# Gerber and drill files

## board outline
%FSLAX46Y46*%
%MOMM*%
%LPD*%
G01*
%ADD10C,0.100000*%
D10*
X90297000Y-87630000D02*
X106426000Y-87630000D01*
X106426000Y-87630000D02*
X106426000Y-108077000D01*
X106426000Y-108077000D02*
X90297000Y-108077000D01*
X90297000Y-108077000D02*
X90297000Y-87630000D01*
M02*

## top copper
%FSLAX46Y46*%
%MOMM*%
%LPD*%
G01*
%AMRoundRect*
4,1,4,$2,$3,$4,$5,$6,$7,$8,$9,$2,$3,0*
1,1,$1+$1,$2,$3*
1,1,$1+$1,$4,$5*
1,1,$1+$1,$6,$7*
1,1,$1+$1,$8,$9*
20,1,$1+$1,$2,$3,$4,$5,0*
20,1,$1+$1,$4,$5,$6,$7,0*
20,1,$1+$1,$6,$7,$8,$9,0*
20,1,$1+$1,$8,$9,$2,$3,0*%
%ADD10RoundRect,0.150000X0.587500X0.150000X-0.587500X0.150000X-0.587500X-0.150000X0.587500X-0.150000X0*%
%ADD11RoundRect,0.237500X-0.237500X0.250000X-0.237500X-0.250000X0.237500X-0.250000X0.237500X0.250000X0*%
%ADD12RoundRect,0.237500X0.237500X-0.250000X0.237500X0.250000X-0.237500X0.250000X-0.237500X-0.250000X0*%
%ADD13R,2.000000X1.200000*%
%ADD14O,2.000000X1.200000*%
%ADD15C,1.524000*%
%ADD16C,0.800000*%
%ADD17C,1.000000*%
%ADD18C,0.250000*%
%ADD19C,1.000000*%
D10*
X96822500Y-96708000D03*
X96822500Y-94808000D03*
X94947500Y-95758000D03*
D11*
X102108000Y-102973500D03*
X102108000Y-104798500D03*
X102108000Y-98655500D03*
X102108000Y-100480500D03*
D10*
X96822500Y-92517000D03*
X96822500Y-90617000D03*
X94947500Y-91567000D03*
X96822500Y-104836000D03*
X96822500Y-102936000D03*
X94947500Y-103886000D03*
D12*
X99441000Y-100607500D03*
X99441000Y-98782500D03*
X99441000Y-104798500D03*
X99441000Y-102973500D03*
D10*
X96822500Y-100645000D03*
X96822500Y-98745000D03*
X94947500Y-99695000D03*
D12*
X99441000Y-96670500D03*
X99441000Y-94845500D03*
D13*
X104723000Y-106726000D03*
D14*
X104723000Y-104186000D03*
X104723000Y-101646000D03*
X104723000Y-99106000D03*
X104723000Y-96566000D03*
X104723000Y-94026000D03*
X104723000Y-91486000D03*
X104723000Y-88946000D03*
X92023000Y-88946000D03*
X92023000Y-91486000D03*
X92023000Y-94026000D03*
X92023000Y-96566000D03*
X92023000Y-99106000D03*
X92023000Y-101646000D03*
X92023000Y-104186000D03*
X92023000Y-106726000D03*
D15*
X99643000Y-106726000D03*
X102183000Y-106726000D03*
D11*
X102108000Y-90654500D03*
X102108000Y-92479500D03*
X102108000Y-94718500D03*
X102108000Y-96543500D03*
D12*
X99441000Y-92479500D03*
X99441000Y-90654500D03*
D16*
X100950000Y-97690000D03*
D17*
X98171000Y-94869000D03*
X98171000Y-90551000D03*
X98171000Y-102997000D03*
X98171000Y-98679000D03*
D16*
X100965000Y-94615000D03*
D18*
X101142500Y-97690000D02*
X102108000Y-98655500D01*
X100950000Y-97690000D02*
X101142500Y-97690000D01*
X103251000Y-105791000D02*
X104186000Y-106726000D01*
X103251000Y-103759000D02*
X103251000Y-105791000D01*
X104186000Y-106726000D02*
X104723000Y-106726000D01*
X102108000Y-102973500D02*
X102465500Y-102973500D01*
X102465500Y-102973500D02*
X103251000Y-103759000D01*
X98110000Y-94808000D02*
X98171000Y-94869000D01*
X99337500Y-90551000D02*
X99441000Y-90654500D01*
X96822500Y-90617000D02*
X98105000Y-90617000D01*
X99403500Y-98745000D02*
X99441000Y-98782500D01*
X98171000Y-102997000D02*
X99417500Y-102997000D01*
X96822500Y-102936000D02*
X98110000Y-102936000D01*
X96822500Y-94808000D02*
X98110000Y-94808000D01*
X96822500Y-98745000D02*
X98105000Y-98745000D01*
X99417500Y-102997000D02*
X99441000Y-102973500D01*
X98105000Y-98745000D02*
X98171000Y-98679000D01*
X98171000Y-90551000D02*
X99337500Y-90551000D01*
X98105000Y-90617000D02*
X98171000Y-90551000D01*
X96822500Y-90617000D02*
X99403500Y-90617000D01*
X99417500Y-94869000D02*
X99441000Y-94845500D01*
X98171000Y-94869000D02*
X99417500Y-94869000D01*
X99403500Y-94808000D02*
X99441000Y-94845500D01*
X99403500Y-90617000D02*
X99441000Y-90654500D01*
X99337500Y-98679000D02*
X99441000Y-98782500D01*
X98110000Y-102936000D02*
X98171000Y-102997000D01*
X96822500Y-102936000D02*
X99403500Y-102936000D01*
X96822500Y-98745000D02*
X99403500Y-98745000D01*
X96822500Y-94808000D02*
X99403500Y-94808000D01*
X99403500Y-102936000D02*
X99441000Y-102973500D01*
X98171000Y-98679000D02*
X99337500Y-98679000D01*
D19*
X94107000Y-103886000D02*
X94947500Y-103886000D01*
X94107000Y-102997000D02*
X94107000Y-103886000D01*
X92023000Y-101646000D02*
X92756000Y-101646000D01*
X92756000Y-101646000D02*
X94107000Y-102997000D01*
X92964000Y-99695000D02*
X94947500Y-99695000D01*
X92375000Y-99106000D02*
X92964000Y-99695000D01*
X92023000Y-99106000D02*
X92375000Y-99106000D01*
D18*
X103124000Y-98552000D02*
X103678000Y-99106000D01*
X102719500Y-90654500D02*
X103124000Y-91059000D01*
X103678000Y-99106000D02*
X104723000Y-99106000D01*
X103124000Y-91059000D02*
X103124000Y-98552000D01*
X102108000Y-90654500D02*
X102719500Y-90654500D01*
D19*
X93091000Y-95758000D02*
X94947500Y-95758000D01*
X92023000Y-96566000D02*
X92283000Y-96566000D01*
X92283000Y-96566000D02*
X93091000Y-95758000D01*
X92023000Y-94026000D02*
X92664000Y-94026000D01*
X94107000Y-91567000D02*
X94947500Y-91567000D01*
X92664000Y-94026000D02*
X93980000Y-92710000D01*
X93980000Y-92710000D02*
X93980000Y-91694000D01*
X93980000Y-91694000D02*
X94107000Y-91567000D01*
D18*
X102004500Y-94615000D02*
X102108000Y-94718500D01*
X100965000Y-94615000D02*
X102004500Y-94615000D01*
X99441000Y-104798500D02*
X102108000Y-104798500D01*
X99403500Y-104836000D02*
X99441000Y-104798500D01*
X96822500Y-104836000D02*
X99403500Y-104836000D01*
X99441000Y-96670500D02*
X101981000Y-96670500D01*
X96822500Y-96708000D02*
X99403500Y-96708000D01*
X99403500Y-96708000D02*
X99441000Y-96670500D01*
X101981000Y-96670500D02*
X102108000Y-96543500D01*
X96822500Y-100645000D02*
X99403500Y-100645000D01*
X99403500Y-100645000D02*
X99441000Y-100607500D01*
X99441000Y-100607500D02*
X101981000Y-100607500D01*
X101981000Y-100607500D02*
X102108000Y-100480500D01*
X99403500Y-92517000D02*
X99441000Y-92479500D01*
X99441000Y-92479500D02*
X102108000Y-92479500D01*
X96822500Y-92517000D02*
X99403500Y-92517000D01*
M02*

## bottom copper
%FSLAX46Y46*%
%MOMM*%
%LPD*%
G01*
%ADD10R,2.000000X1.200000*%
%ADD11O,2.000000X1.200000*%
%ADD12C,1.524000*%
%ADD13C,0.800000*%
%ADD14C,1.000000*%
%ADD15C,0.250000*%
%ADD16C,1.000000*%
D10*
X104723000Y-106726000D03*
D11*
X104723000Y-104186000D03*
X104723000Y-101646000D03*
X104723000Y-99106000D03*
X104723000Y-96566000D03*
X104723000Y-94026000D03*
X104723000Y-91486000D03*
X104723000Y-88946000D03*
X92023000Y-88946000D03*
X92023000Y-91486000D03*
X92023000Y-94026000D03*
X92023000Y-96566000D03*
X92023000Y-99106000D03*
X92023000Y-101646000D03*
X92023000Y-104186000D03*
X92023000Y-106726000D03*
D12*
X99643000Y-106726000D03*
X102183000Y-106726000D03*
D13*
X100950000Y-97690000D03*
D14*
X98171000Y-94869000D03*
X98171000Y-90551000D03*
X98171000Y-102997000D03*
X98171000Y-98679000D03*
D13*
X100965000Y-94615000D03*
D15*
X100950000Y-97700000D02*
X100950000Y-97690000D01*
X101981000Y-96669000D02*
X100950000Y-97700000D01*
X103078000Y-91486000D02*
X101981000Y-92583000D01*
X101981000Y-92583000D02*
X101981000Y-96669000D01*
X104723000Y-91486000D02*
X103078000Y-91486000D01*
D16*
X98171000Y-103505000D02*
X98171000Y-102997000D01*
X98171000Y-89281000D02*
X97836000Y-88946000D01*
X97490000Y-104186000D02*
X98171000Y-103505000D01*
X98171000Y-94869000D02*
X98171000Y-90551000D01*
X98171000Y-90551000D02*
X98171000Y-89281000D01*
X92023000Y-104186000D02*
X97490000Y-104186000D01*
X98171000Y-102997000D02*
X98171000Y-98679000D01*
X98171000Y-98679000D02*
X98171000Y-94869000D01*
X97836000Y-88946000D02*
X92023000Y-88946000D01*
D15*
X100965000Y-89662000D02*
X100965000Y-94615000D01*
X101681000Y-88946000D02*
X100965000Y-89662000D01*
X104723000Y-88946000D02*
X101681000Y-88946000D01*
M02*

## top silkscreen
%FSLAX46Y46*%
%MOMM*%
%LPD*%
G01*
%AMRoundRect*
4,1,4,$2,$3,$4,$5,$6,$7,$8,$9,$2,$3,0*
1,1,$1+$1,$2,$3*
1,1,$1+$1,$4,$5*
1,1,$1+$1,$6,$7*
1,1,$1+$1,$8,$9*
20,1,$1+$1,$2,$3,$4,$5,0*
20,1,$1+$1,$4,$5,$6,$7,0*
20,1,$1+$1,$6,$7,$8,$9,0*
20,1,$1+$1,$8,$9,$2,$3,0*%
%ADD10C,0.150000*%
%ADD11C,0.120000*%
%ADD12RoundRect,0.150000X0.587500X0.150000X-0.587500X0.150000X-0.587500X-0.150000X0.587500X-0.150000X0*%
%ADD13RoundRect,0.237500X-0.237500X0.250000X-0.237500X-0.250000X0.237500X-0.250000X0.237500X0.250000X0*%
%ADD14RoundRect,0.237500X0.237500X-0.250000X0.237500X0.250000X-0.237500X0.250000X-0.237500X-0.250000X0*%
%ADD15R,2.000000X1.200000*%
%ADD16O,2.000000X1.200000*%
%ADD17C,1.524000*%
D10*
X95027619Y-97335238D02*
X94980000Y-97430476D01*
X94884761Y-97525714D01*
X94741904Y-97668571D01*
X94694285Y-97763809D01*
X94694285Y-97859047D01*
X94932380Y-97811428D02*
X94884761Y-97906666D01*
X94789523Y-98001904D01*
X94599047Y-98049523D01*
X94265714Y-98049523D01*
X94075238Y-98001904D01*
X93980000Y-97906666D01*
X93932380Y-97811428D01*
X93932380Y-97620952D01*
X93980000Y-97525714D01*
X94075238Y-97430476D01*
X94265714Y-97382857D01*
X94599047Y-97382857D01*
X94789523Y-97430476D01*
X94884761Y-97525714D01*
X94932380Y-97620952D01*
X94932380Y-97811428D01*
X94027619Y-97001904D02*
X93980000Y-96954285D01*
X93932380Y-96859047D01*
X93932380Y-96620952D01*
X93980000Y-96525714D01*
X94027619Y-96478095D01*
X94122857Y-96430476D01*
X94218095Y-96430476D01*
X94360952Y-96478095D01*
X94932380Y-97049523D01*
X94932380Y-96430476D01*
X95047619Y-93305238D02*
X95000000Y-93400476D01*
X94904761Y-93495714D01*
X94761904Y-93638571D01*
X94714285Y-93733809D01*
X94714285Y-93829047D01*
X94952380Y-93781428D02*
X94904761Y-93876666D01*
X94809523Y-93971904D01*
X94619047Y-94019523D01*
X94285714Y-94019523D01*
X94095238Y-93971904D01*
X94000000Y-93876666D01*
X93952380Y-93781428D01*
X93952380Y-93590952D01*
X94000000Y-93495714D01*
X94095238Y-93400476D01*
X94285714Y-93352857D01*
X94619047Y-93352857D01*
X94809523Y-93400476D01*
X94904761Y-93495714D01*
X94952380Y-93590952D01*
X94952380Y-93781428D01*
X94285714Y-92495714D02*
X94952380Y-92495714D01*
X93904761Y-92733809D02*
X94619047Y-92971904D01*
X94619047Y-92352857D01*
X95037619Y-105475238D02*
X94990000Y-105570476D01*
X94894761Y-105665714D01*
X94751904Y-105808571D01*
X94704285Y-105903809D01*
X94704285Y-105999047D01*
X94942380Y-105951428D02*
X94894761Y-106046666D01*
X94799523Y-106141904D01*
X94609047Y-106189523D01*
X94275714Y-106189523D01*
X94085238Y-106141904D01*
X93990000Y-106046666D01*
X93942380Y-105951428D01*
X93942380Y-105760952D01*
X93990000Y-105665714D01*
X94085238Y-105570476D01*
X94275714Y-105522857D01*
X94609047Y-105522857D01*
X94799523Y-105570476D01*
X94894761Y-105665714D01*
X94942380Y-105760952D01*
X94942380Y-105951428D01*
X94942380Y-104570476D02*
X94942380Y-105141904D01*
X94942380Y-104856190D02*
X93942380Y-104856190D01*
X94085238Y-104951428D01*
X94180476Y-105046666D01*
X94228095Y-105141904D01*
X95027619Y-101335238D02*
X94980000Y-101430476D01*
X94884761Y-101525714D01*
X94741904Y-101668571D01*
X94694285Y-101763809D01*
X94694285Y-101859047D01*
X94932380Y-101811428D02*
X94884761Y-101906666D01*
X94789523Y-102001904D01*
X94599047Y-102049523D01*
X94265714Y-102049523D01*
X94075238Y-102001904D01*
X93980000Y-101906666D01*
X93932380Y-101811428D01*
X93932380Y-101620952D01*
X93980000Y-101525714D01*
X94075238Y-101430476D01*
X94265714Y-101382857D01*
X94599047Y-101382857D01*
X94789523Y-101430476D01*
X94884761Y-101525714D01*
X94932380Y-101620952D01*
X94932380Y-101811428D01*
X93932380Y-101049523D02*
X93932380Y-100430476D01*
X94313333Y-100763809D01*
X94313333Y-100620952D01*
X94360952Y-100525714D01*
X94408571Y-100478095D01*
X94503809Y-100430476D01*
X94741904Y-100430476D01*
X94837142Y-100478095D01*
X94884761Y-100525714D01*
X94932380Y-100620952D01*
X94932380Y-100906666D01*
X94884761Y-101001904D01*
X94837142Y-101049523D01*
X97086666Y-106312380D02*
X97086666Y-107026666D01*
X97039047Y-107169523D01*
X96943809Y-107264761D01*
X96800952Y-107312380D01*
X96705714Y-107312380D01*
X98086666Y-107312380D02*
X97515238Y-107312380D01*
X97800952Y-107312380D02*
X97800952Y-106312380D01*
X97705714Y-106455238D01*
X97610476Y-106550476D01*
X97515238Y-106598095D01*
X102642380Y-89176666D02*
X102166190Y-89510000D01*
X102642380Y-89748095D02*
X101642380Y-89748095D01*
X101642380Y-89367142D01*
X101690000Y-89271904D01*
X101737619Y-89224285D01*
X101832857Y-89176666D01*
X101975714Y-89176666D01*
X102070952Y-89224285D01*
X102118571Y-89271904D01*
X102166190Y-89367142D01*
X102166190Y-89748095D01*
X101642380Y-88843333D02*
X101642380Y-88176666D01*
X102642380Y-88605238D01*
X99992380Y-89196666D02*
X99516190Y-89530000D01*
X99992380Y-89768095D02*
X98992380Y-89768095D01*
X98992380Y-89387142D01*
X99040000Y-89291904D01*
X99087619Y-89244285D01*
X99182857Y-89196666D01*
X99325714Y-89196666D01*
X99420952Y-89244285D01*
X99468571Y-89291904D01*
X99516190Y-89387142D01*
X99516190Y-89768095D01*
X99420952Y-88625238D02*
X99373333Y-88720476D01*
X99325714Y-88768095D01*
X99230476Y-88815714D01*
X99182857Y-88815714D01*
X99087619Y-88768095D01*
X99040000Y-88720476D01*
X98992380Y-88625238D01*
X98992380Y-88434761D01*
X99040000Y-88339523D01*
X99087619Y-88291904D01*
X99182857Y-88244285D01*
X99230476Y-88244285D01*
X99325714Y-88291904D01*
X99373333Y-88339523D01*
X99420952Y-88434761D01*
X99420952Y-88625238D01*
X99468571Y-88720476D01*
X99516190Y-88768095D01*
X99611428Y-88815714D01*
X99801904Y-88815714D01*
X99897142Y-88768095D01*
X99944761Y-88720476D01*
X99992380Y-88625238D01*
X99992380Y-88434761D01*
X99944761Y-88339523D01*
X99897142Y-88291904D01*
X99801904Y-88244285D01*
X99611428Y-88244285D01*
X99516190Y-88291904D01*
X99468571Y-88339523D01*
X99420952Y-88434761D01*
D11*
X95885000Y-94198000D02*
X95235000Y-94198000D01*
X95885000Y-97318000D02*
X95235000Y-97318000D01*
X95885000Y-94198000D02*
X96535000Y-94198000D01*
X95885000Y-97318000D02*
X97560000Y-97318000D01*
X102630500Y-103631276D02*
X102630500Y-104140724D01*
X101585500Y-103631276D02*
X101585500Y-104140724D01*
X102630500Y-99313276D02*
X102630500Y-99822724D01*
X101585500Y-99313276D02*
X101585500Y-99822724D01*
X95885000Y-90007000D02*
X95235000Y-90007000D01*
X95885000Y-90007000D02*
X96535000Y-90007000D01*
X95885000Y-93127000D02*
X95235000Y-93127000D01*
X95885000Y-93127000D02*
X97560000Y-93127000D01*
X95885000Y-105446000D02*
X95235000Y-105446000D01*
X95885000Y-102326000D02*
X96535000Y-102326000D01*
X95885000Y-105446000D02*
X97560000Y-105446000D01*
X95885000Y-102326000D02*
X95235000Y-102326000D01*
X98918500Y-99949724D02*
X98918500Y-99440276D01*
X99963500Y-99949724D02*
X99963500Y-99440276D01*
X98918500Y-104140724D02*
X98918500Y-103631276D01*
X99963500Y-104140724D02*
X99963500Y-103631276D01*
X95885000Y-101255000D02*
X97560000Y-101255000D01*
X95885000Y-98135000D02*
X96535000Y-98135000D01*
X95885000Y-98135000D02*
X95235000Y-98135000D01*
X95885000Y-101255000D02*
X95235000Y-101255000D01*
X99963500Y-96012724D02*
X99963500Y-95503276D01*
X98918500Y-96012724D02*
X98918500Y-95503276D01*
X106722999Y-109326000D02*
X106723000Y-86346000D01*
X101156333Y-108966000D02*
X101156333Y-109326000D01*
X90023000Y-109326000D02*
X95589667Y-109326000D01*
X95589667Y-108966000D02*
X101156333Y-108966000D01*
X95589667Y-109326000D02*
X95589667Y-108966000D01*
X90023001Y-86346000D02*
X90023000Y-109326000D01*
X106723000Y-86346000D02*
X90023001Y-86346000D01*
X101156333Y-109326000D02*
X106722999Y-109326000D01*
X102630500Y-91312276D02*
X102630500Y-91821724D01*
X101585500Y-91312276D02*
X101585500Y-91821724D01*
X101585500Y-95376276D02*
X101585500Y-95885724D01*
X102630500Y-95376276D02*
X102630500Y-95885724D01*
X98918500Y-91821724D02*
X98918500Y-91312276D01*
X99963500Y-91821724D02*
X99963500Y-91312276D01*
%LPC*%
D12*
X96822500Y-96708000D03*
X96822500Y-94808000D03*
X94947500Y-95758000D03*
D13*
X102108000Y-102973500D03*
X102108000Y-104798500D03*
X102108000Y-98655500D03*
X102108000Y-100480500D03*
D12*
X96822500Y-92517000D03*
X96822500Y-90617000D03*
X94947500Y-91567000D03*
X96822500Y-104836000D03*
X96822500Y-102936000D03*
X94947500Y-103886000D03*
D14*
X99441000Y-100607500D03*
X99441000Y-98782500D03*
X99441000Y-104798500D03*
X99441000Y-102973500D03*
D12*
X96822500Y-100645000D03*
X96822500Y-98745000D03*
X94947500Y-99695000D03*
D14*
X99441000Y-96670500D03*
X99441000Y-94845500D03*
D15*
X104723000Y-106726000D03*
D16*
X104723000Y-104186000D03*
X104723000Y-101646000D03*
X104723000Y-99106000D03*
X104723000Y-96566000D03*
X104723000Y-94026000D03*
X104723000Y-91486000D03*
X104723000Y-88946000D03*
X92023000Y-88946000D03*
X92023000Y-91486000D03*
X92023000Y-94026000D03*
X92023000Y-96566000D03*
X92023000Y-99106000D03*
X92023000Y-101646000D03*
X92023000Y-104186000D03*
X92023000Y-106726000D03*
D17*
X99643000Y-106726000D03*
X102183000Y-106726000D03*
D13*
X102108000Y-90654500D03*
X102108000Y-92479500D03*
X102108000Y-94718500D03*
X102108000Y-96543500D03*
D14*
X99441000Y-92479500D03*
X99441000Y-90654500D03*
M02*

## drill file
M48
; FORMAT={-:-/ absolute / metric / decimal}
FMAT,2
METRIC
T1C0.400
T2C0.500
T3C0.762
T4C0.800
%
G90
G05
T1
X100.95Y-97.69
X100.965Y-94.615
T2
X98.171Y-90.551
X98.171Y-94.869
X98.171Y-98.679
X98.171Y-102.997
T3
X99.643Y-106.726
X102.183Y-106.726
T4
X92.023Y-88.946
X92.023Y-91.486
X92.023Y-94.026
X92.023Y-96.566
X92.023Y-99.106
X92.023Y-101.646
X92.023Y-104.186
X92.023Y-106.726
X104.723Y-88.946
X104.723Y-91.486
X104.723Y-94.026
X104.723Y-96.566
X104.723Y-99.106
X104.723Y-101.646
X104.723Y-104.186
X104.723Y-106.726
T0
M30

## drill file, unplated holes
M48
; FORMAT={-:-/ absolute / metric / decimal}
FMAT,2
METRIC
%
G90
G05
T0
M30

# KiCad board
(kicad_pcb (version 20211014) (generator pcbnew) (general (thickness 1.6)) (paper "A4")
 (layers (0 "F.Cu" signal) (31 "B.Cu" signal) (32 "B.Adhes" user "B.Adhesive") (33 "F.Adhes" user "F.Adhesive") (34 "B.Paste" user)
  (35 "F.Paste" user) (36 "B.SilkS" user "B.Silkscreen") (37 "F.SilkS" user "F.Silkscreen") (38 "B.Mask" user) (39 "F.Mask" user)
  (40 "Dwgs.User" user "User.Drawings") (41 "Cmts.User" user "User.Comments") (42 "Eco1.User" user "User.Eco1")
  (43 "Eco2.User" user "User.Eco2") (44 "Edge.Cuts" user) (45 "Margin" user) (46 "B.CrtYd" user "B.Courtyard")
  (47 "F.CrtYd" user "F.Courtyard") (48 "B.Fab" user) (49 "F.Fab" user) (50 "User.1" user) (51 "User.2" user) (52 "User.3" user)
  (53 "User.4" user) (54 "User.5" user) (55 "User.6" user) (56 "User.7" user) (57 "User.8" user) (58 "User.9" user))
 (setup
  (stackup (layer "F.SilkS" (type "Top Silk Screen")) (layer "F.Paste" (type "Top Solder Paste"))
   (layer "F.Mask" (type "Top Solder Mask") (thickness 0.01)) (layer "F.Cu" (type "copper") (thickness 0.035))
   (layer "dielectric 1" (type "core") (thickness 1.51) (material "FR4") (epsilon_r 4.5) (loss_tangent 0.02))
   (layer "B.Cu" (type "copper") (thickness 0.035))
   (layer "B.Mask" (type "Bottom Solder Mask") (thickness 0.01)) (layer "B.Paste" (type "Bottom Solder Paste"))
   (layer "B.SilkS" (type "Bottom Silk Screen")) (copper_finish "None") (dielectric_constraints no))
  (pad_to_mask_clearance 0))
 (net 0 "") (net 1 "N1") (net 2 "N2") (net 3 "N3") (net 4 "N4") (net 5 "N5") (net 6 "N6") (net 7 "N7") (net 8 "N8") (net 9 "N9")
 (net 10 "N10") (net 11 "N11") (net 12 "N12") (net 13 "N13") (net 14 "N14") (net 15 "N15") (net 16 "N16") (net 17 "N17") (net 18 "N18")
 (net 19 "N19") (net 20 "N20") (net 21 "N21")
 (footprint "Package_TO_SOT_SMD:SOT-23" (layer "F.Cu") (at 95.885 95.758 180)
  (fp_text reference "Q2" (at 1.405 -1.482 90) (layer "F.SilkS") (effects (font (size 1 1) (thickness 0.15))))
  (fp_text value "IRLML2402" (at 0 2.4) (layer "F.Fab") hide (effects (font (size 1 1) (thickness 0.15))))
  (fp_line (start 0 1.56) (end 0.65 1.56) (layer "F.SilkS") (width 0.12))
  (fp_line (start 0 -1.56) (end 0.65 -1.56) (layer "F.SilkS") (width 0.12))
  (fp_line (start 0 1.56) (end -0.65 1.56) (layer "F.SilkS") (width 0.12))
  (fp_line (start 0 -1.56) (end -1.675 -1.56) (layer "F.SilkS") (width 0.12))
  (pad "1" smd roundrect locked (at -0.9375 -0.95 180) (size 1.475 0.6) (layers "F.Cu" "F.Paste" "F.Mask") (roundrect_rratio 0.25)
   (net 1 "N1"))
  (pad "2" smd roundrect locked (at -0.9375 0.95 180) (size 1.475 0.6) (layers "F.Cu" "F.Paste" "F.Mask") (roundrect_rratio 0.25)
   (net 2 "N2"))
  (pad "3" smd roundrect locked (at 0.9375 0 180) (size 1.475 0.6) (layers "F.Cu" "F.Paste" "F.Mask") (roundrect_rratio 0.25) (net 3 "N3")))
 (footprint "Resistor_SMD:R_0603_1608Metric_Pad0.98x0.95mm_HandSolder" (layer "F.Cu") (at 102.108 103.886 -90)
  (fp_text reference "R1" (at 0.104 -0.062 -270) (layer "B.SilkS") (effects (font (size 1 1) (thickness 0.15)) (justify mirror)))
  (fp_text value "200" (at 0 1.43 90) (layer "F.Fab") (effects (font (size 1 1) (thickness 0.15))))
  (fp_line (start -0.254724 -0.5225) (end 0.254724 -0.5225) (layer "F.SilkS") (width 0.12))
  (fp_line (start -0.254724 0.5225) (end 0.254724 0.5225) (layer "F.SilkS") (width 0.12))
  (pad "1" smd roundrect locked (at -0.9125 0 270) (size 0.975 0.95) (layers "F.Cu" "F.Paste" "F.Mask") (roundrect_rratio 0.25) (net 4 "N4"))
  (pad "2" smd roundrect locked (at 0.9125 0 270) (size 0.975 0.95) (layers "F.Cu" "F.Paste" "F.Mask") (roundrect_rratio 0.25) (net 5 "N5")))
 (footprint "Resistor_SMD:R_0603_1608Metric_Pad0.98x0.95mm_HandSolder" (layer "F.Cu") (at 102.108 99.568 -90)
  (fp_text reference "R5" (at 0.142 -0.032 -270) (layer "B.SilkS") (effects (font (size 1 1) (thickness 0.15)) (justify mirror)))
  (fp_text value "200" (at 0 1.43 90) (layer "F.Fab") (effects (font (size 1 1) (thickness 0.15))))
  (fp_line (start -0.254724 -0.5225) (end 0.254724 -0.5225) (layer "F.SilkS") (width 0.12))
  (fp_line (start -0.254724 0.5225) (end 0.254724 0.5225) (layer "F.SilkS") (width 0.12))
  (pad "1" smd roundrect locked (at -0.9125 0 270) (size 0.975 0.95) (layers "F.Cu" "F.Paste" "F.Mask") (roundrect_rratio 0.25) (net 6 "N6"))
  (pad "2" smd roundrect locked (at 0.9125 0 270) (size 0.975 0.95) (layers "F.Cu" "F.Paste" "F.Mask") (roundrect_rratio 0.25) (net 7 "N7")))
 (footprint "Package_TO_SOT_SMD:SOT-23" (layer "F.Cu") (at 95.885 91.567 180)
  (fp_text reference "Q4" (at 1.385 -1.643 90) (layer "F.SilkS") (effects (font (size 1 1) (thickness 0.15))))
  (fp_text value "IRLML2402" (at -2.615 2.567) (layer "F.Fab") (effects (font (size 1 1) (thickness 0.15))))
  (fp_line (start 0 1.56) (end 0.65 1.56) (layer "F.SilkS") (width 0.12))
  (fp_line (start 0 1.56) (end -0.65 1.56) (layer "F.SilkS") (width 0.12))
  (fp_line (start 0 -1.56) (end 0.65 -1.56) (layer "F.SilkS") (width 0.12))
  (fp_line (start 0 -1.56) (end -1.675 -1.56) (layer "F.SilkS") (width 0.12))
  (pad "1" smd roundrect locked (at -0.9375 -0.95 180) (size 1.475 0.6) (layers "F.Cu" "F.Paste" "F.Mask") (roundrect_rratio 0.25)
   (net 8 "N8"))
  (pad "2" smd roundrect locked (at -0.9375 0.95 180) (size 1.475 0.6) (layers "F.Cu" "F.Paste" "F.Mask") (roundrect_rratio 0.25)
   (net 2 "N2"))
  (pad "3" smd roundrect locked (at 0.9375 0 180) (size 1.475 0.6) (layers "F.Cu" "F.Paste" "F.Mask") (roundrect_rratio 0.25) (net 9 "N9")))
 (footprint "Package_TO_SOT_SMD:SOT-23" (layer "F.Cu") (at 95.885 103.886 180)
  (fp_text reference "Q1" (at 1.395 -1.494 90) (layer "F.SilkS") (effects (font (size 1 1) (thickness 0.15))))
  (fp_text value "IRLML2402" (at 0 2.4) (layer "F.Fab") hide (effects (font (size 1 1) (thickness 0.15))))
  (fp_line (start 0 -1.56) (end 0.65 -1.56) (layer "F.SilkS") (width 0.12))
  (fp_line (start 0 1.56) (end -0.65 1.56) (layer "F.SilkS") (width 0.12))
  (fp_line (start 0 -1.56) (end -1.675 -1.56) (layer "F.SilkS") (width 0.12))
  (fp_line (start 0 1.56) (end 0.65 1.56) (layer "F.SilkS") (width 0.12))
  (pad "1" smd roundrect locked (at -0.9375 -0.95 180) (size 1.475 0.6) (layers "F.Cu" "F.Paste" "F.Mask") (roundrect_rratio 0.25)
   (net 5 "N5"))
  (pad "2" smd roundrect locked (at -0.9375 0.95 180) (size 1.475 0.6) (layers "F.Cu" "F.Paste" "F.Mask") (roundrect_rratio 0.25)
   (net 2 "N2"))
  (pad "3" smd roundrect locked (at 0.9375 0 180) (size 1.475 0.6) (layers "F.Cu" "F.Paste" "F.Mask") (roundrect_rratio 0.25) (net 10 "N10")))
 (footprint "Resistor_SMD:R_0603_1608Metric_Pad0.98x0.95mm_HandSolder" (layer "F.Cu") (at 99.441 99.695 90)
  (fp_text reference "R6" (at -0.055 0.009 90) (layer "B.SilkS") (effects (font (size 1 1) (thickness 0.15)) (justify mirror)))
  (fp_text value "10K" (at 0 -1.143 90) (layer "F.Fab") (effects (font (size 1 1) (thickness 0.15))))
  (fp_line (start -0.254724 -0.5225) (end 0.254724 -0.5225) (layer "F.SilkS") (width 0.12))
  (fp_line (start -0.254724 0.5225) (end 0.254724 0.5225) (layer "F.SilkS") (width 0.12))
  (pad "1" smd roundrect locked (at -0.9125 0 90) (size 0.975 0.95) (layers "F.Cu" "F.Paste" "F.Mask") (roundrect_rratio 0.25) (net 7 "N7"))
  (pad "2" smd roundrect locked (at 0.9125 0 90) (size 0.975 0.95) (layers "F.Cu" "F.Paste" "F.Mask") (roundrect_rratio 0.25) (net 2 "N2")))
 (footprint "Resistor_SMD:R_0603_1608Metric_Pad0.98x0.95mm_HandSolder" (layer "F.Cu") (at 99.441 103.886 90)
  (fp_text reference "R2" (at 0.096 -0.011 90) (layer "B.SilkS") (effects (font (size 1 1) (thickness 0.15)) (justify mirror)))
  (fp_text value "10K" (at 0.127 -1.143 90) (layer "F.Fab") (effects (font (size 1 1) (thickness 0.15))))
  (fp_line (start -0.254724 -0.5225) (end 0.254724 -0.5225) (layer "F.SilkS") (width 0.12))
  (fp_line (start -0.254724 0.5225) (end 0.254724 0.5225) (layer "F.SilkS") (width 0.12))
  (pad "1" smd roundrect locked (at -0.9125 0 90) (size 0.975 0.95) (layers "F.Cu" "F.Paste" "F.Mask") (roundrect_rratio 0.25) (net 5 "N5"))
  (pad "2" smd roundrect locked (at 0.9125 0 90) (size 0.975 0.95) (layers "F.Cu" "F.Paste" "F.Mask") (roundrect_rratio 0.25) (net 2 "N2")))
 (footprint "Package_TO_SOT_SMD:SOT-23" (layer "F.Cu") (at 95.885 99.695 180)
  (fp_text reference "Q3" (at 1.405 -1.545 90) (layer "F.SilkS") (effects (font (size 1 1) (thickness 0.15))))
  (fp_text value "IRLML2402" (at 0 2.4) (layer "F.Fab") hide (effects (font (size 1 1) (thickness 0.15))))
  (fp_line (start 0 -1.56) (end -1.675 -1.56) (layer "F.SilkS") (width 0.12))
  (fp_line (start 0 1.56) (end -0.65 1.56) (layer "F.SilkS") (width 0.12))
  (fp_line (start 0 1.56) (end 0.65 1.56) (layer "F.SilkS") (width 0.12))
  (fp_line (start 0 -1.56) (end 0.65 -1.56) (layer "F.SilkS") (width 0.12))
  (pad "1" smd roundrect locked (at -0.9375 -0.95 180) (size 1.475 0.6) (layers "F.Cu" "F.Paste" "F.Mask") (roundrect_rratio 0.25)
   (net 7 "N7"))
  (pad "2" smd roundrect locked (at -0.9375 0.95 180) (size 1.475 0.6) (layers "F.Cu" "F.Paste" "F.Mask") (roundrect_rratio 0.25)
   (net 2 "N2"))
  (pad "3" smd roundrect locked (at 0.9375 0 180) (size 1.475 0.6) (layers "F.Cu" "F.Paste" "F.Mask") (roundrect_rratio 0.25) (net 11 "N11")))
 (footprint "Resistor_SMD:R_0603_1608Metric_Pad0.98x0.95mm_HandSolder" (layer "F.Cu") (at 99.441 95.758 90)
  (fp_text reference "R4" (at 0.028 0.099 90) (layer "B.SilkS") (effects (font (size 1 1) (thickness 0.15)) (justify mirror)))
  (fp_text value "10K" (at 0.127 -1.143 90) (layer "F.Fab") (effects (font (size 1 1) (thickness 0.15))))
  (fp_line (start -0.254724 0.5225) (end 0.254724 0.5225) (layer "F.SilkS") (width 0.12))
  (fp_line (start -0.254724 -0.5225) (end 0.254724 -0.5225) (layer "F.SilkS") (width 0.12))
  (pad "1" smd roundrect locked (at -0.9125 0 90) (size 0.975 0.95) (layers "F.Cu" "F.Paste" "F.Mask") (roundrect_rratio 0.25) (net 1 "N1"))
  (pad "2" smd roundrect locked (at 0.9125 0 90) (size 0.975 0.95) (layers "F.Cu" "F.Paste" "F.Mask") (roundrect_rratio 0.25) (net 2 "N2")))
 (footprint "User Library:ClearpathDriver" (layer "F.Cu") (at 98.373 97.836)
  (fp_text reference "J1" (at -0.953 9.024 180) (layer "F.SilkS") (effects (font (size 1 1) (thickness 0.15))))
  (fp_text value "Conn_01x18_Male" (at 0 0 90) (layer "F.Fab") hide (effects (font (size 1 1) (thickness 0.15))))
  (fp_line (start 8.349999 11.49) (end 8.35 -11.49) (layer "F.SilkS") (width 0.12))
  (fp_line (start 2.783333 11.13) (end 2.783333 11.49) (layer "F.SilkS") (width 0.12))
  (fp_line (start -8.35 11.49) (end -2.783333 11.49) (layer "F.SilkS") (width 0.12))
  (fp_line (start -2.783333 11.13) (end 2.783333 11.13) (layer "F.SilkS") (width 0.12))
  (fp_line (start -2.783333 11.49) (end -2.783333 11.13) (layer "F.SilkS") (width 0.12))
  (fp_line (start -8.349999 -11.49) (end -8.35 11.49) (layer "F.SilkS") (width 0.12))
  (fp_line (start 8.35 -11.49) (end -8.349999 -11.49) (layer "F.SilkS") (width 0.12))
  (fp_line (start 2.783333 11.49) (end 8.349999 11.49) (layer "F.SilkS") (width 0.12))
  (pad "1" thru_hole rect locked (at 6.35 8.89 90) (size 1.2 2) (drill 0.8) (layers *.Cu *.Mask) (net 4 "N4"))
  (pad "2" thru_hole oval locked (at 6.35 6.35 90) (size 1.2 2) (drill 0.8) (layers *.Cu *.Mask) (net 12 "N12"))
  (pad "3" thru_hole oval locked (at 6.35 3.81 90) (size 1.2 2) (drill 0.8) (layers *.Cu *.Mask) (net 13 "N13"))
  (pad "4" thru_hole oval locked (at 6.35 1.27 90) (size 1.2 2) (drill 0.8) (layers *.Cu *.Mask) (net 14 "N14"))
  (pad "5" thru_hole oval locked (at 6.35 -1.27 90) (size 1.2 2) (drill 0.8) (layers *.Cu *.Mask) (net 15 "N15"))
  (pad "6" thru_hole oval locked (at 6.35 -3.81 90) (size 1.2 2) (drill 0.8) (layers *.Cu *.Mask) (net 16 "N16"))
  (pad "7" thru_hole oval locked (at 6.35 -6.35 90) (size 1.2 2) (drill 0.8) (layers *.Cu *.Mask) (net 6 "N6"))
  (pad "8" thru_hole oval locked (at 6.35 -8.89 90) (size 1.2 2) (drill 0.8) (layers *.Cu *.Mask) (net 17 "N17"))
  (pad "9" thru_hole oval locked (at -6.35 -8.89 90) (size 1.2 2) (drill 0.8) (layers *.Cu *.Mask) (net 2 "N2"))
  (pad "10" thru_hole oval locked (at -6.35 -6.35 90) (size 1.2 2) (drill 0.8) (layers *.Cu *.Mask) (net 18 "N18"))
  (pad "11" thru_hole oval locked (at -6.35 -3.81 90) (size 1.2 2) (drill 0.8) (layers *.Cu *.Mask) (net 9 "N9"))
  (pad "12" thru_hole oval locked (at -6.35 -1.27 90) (size 1.2 2) (drill 0.8) (layers *.Cu *.Mask) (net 3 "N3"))
  (pad "13" thru_hole oval locked (at -6.35 1.27 90) (size 1.2 2) (drill 0.8) (layers *.Cu *.Mask) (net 11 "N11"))
  (pad "14" thru_hole oval locked (at -6.35 3.81 90) (size 1.2 2) (drill 0.8) (layers *.Cu *.Mask) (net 10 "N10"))
  (pad "15" thru_hole oval locked (at -6.35 6.35 90) (size 1.2 2) (drill 0.8) (layers *.Cu *.Mask) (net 2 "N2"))
  (pad "16" thru_hole oval locked (at -6.35 8.89 90) (size 1.2 2) (drill 0.8) (layers *.Cu *.Mask) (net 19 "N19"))
  (pad "17" thru_hole circle locked (at 1.27 8.89) (size 1.524 1.524) (drill 0.762) (layers *.Cu *.Mask) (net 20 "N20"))
  (pad "18" thru_hole circle locked (at 3.81 8.89) (size 1.524 1.524) (drill 0.762) (layers *.Cu *.Mask) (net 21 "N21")))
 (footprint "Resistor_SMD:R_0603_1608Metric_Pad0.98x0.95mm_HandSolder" (layer "F.Cu") (at 102.108 91.567 -90)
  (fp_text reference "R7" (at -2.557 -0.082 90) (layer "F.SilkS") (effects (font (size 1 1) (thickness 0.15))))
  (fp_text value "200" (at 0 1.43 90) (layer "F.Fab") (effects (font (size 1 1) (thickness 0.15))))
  (fp_line (start -0.254724 -0.5225) (end 0.254724 -0.5225) (layer "F.SilkS") (width 0.12))
  (fp_line (start -0.254724 0.5225) (end 0.254724 0.5225) (layer "F.SilkS") (width 0.12))
  (pad "1" smd roundrect locked (at -0.9125 0 270) (size 0.975 0.95) (layers "F.Cu" "F.Paste" "F.Mask") (roundrect_rratio 0.25)
   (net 14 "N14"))
  (pad "2" smd roundrect locked (at 0.9125 0 270) (size 0.975 0.95) (layers "F.Cu" "F.Paste" "F.Mask") (roundrect_rratio 0.25) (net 8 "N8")))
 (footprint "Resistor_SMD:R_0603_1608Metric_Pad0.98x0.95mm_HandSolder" (layer "F.Cu") (at 102.108 95.631 -90)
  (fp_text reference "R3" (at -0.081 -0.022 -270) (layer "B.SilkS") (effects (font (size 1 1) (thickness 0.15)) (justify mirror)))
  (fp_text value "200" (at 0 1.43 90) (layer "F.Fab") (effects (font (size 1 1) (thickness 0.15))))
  (fp_line (start -0.254724 0.5225) (end 0.254724 0.5225) (layer "F.SilkS") (width 0.12))
  (fp_line (start -0.254724 -0.5225) (end 0.254724 -0.5225) (layer "F.SilkS") (width 0.12))
  (pad "1" smd roundrect locked (at -0.9125 0 270) (size 0.975 0.95) (layers "F.Cu" "F.Paste" "F.Mask") (roundrect_rratio 0.25)
   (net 17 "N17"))
  (pad "2" smd roundrect locked (at 0.9125 0 270) (size 0.975 0.95) (layers "F.Cu" "F.Paste" "F.Mask") (roundrect_rratio 0.25) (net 1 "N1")))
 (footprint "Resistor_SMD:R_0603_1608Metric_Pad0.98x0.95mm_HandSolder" (layer "F.Cu") (at 99.441 91.567 90)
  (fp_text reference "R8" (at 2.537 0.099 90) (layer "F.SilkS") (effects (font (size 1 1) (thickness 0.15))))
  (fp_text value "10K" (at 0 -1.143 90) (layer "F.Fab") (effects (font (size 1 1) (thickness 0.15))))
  (fp_line (start -0.254724 -0.5225) (end 0.254724 -0.5225) (layer "F.SilkS") (width 0.12))
  (fp_line (start -0.254724 0.5225) (end 0.254724 0.5225) (layer "F.SilkS") (width 0.12))
  (pad "1" smd roundrect locked (at -0.9125 0 90) (size 0.975 0.95) (layers "F.Cu" "F.Paste" "F.Mask") (roundrect_rratio 0.25) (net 8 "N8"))
  (pad "2" smd roundrect locked (at 0.9125 0 90) (size 0.975 0.95) (layers "F.Cu" "F.Paste" "F.Mask") (roundrect_rratio 0.25) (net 2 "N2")))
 (gr_rect (start 90.297 87.63) (end 106.426 108.077) (layer "Edge.Cuts") (width 0.1) (fill none))
 (segment (start 103.251 105.791) (end 104.186 106.726) (width 0.25) (layer "F.Cu") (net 4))
 (segment (start 103.251 103.759) (end 103.251 105.791) (width 0.25) (layer "F.Cu") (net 4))
 (segment (start 104.186 106.726) (end 104.723 106.726) (width 0.25) (layer "F.Cu") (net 4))
 (segment (start 102.108 102.9735) (end 102.4655 102.9735) (width 0.25) (layer "F.Cu") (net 4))
 (segment (start 102.4655 102.9735) (end 103.251 103.759) (width 0.25) (layer "F.Cu") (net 4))
 (segment (start 98.11 94.808) (end 98.171 94.869) (width 0.25) (layer "F.Cu") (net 2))
 (segment (start 99.3375 90.551) (end 99.441 90.6545) (width 0.25) (layer "F.Cu") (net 2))
 (segment (start 96.8225 90.617) (end 98.105 90.617) (width 0.25) (layer "F.Cu") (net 2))
 (segment (start 99.4035 98.745) (end 99.441 98.7825) (width 0.25) (layer "F.Cu") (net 2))
 (segment (start 98.171 102.997) (end 99.4175 102.997) (width 0.25) (layer "F.Cu") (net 2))
 (segment (start 96.8225 102.936) (end 98.11 102.936) (width 0.25) (layer "F.Cu") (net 2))
 (segment (start 96.8225 94.808) (end 98.11 94.808) (width 0.25) (layer "F.Cu") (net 2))
 (segment (start 96.8225 98.745) (end 98.105 98.745) (width 0.25) (layer "F.Cu") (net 2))
 (segment (start 99.4175 102.997) (end 99.441 102.9735) (width 0.25) (layer "F.Cu") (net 2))
 (segment (start 98.105 98.745) (end 98.171 98.679) (width 0.25) (layer "F.Cu") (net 2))
 (segment (start 98.171 90.551) (end 99.3375 90.551) (width 0.25) (layer "F.Cu") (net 2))
 (segment (start 98.105 90.617) (end 98.171 90.551) (width 0.25) (layer "F.Cu") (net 2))
 (segment (start 96.8225 90.617) (end 99.4035 90.617) (width 0.25) (layer "F.Cu") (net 2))
 (segment (start 99.4175 94.869) (end 99.441 94.8455) (width 0.25) (layer "F.Cu") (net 2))
 (segment (start 98.171 94.869) (end 99.4175 94.869) (width 0.25) (layer "F.Cu") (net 2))
 (segment (start 99.4035 94.808) (end 99.441 94.8455) (width 0.25) (layer "F.Cu") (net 2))
 (segment (start 99.4035 90.617) (end 99.441 90.6545) (width 0.25) (layer "F.Cu") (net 2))
 (segment (start 99.3375 98.679) (end 99.441 98.7825) (width 0.25) (layer "F.Cu") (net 2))
 (segment (start 98.11 102.936) (end 98.171 102.997) (width 0.25) (layer "F.Cu") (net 2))
 (segment (start 96.8225 102.936) (end 99.4035 102.936) (width 0.25) (layer "F.Cu") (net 2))
 (segment (start 96.8225 98.745) (end 99.4035 98.745) (width 0.25) (layer "F.Cu") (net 2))
 (segment (start 96.8225 94.808) (end 99.4035 94.808) (width 0.25) (layer "F.Cu") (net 2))
 (segment (start 99.4035 102.936) (end 99.441 102.9735) (width 0.25) (layer "F.Cu") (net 2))
 (segment (start 98.171 98.679) (end 99.3375 98.679) (width 0.25) (layer "F.Cu") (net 2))
 (via (at 98.171 94.869) (size 1) (drill 0.5) (layers "F.Cu" "B.Cu") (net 2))
 (via (at 98.171 90.551) (size 1) (drill 0.5) (layers "F.Cu" "B.Cu") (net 2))
 (via (at 98.171 102.997) (size 1) (drill 0.5) (layers "F.Cu" "B.Cu") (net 2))
 (via (at 98.171 98.679) (size 1) (drill 0.5) (layers "F.Cu" "B.Cu") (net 2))
 (segment (start 98.171 103.505) (end 98.171 102.997) (width 1) (layer "B.Cu") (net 2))
 (segment (start 98.171 89.281) (end 97.836 88.946) (width 1) (layer "B.Cu") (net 2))
 (segment (start 97.49 104.186) (end 98.171 103.505) (width 1) (layer "B.Cu") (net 2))
 (segment (start 98.171 94.869) (end 98.171 90.551) (width 1) (layer "B.Cu") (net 2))
 (segment (start 98.171 90.551) (end 98.171 89.281) (width 1) (layer "B.Cu") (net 2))
 (segment (start 92.023 104.186) (end 97.49 104.186) (width 1) (layer "B.Cu") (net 2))
 (segment (start 98.171 102.997) (end 98.171 98.679) (width 1) (layer "B.Cu") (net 2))
 (segment (start 98.171 98.679) (end 98.171 94.869) (width 1) (layer "B.Cu") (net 2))
 (segment (start 97.836 88.946) (end 92.023 88.946) (width 1) (layer "B.Cu") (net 2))
 (segment (start 94.107 103.886) (end 94.9475 103.886) (width 1) (layer "F.Cu") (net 10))
 (segment (start 94.107 102.997) (end 94.107 103.886) (width 1) (layer "F.Cu") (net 10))
 (segment (start 92.023 101.646) (end 92.756 101.646) (width 1) (layer "F.Cu") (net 10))
 (segment (start 92.756 101.646) (end 94.107 102.997) (width 1) (layer "F.Cu") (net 10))
 (segment (start 92.964 99.695) (end 94.9475 99.695) (width 1) (layer "F.Cu") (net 11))
 (segment (start 92.375 99.106) (end 92.964 99.695) (width 1) (layer "F.Cu") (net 11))
 (segment (start 92.023 99.106) (end 92.375 99.106) (width 1) (layer "F.Cu") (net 11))
 (segment (start 103.124 98.552) (end 103.678 99.106) (width 0.25) (layer "F.Cu") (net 14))
 (segment (start 102.7195 90.6545) (end 103.124 91.059) (width 0.25) (layer "F.Cu") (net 14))
 (segment (start 103.678 99.106) (end 104.723 99.106) (width 0.25) (layer "F.Cu") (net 14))
 (segment (start 103.124 91.059) (end 103.124 98.552) (width 0.25) (layer "F.Cu") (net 14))
 (segment (start 102.108 90.6545) (end 102.7195 90.6545) (width 0.25) (layer "F.Cu") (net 14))
 (segment (start 93.091 95.758) (end 94.9475 95.758) (width 1) (layer "F.Cu") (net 3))
 (segment (start 92.023 96.566) (end 92.283 96.566) (width 1) (layer "F.Cu") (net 3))
 (segment (start 92.283 96.566) (end 93.091 95.758) (width 1) (layer "F.Cu") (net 3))
 (segment (start 92.023 94.026) (end 92.664 94.026) (width 1) (layer "F.Cu") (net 9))
 (segment (start 94.107 91.567) (end 94.9475 91.567) (width 1) (layer "F.Cu") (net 9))
 (segment (start 92.664 94.026) (end 93.98 92.71) (width 1) (layer "F.Cu") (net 9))
 (segment (start 93.98 92.71) (end 93.98 91.694) (width 1) (layer "F.Cu") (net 9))
 (segment (start 93.98 91.694) (end 94.107 91.567) (width 1) (layer "F.Cu") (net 9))
 (segment (start 101.1425 97.69) (end 102.108 98.6555) (width 0.25) (layer "F.Cu") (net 6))
 (segment (start 100.95 97.69) (end 101.1425 97.69) (width 0.25) (layer "F.Cu") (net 6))
 (via (at 100.95 97.69) (size 0.8) (drill 0.4) (layers "F.Cu" "B.Cu") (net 6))
 (segment (start 101.981 92.583) (end 101.981 96.669) (width 0.25) (layer "B.Cu") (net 6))
 (segment (start 101.981 96.669) (end 100.95 97.7) (width 0.25) (layer "B.Cu") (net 6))
 (segment (start 103.078 91.486) (end 101.981 92.583) (width 0.25) (layer "B.Cu") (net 6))
 (segment (start 100.95 97.7) (end 100.95 97.69) (width 0.25) (layer "B.Cu") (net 6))
 (segment (start 104.723 91.486) (end 103.078 91.486) (width 0.25) (layer "B.Cu") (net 6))
 (segment (start 102.0045 94.615) (end 102.108 94.7185) (width 0.25) (layer "F.Cu") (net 17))
 (segment (start 100.965 94.615) (end 102.0045 94.615) (width 0.25) (layer "F.Cu") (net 17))
 (via (at 100.965 94.615) (size 0.8) (drill 0.4) (layers "F.Cu" "B.Cu") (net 17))
 (segment (start 100.965 89.662) (end 100.965 94.615) (width 0.25) (layer "B.Cu") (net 17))
 (segment (start 101.681 88.946) (end 100.965 89.662) (width 0.25) (layer "B.Cu") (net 17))
 (segment (start 104.723 88.946) (end 101.681 88.946) (width 0.25) (layer "B.Cu") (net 17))
 (segment (start 99.441 104.7985) (end 102.108 104.7985) (width 0.25) (layer "F.Cu") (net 5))
 (segment (start 99.4035 104.836) (end 99.441 104.7985) (width 0.25) (layer "F.Cu") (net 5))
 (segment (start 96.8225 104.836) (end 99.4035 104.836) (width 0.25) (layer "F.Cu") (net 5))
 (segment (start 99.441 96.6705) (end 101.981 96.6705) (width 0.25) (layer "F.Cu") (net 1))
 (segment (start 96.8225 96.708) (end 99.4035 96.708) (width 0.25) (layer "F.Cu") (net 1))
 (segment (start 99.4035 96.708) (end 99.441 96.6705) (width 0.25) (layer "F.Cu") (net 1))
 (segment (start 101.981 96.6705) (end 102.108 96.5435) (width 0.25) (layer "F.Cu") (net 1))
 (segment (start 96.8225 100.645) (end 99.4035 100.645) (width 0.25) (layer "F.Cu") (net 7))
 (segment (start 99.4035 100.645) (end 99.441 100.6075) (width 0.25) (layer "F.Cu") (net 7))
 (segment (start 99.441 100.6075) (end 101.981 100.6075) (width 0.25) (layer "F.Cu") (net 7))
 (segment (start 101.981 100.6075) (end 102.108 100.4805) (width 0.25) (layer "F.Cu") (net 7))
 (segment (start 99.4035 92.517) (end 99.441 92.4795) (width 0.25) (layer "F.Cu") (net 8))
 (segment (start 99.441 92.4795) (end 102.108 92.4795) (width 0.25) (layer "F.Cu") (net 8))
 (segment (start 96.8225 92.517) (end 99.4035 92.517) (width 0.25) (layer "F.Cu") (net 8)))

